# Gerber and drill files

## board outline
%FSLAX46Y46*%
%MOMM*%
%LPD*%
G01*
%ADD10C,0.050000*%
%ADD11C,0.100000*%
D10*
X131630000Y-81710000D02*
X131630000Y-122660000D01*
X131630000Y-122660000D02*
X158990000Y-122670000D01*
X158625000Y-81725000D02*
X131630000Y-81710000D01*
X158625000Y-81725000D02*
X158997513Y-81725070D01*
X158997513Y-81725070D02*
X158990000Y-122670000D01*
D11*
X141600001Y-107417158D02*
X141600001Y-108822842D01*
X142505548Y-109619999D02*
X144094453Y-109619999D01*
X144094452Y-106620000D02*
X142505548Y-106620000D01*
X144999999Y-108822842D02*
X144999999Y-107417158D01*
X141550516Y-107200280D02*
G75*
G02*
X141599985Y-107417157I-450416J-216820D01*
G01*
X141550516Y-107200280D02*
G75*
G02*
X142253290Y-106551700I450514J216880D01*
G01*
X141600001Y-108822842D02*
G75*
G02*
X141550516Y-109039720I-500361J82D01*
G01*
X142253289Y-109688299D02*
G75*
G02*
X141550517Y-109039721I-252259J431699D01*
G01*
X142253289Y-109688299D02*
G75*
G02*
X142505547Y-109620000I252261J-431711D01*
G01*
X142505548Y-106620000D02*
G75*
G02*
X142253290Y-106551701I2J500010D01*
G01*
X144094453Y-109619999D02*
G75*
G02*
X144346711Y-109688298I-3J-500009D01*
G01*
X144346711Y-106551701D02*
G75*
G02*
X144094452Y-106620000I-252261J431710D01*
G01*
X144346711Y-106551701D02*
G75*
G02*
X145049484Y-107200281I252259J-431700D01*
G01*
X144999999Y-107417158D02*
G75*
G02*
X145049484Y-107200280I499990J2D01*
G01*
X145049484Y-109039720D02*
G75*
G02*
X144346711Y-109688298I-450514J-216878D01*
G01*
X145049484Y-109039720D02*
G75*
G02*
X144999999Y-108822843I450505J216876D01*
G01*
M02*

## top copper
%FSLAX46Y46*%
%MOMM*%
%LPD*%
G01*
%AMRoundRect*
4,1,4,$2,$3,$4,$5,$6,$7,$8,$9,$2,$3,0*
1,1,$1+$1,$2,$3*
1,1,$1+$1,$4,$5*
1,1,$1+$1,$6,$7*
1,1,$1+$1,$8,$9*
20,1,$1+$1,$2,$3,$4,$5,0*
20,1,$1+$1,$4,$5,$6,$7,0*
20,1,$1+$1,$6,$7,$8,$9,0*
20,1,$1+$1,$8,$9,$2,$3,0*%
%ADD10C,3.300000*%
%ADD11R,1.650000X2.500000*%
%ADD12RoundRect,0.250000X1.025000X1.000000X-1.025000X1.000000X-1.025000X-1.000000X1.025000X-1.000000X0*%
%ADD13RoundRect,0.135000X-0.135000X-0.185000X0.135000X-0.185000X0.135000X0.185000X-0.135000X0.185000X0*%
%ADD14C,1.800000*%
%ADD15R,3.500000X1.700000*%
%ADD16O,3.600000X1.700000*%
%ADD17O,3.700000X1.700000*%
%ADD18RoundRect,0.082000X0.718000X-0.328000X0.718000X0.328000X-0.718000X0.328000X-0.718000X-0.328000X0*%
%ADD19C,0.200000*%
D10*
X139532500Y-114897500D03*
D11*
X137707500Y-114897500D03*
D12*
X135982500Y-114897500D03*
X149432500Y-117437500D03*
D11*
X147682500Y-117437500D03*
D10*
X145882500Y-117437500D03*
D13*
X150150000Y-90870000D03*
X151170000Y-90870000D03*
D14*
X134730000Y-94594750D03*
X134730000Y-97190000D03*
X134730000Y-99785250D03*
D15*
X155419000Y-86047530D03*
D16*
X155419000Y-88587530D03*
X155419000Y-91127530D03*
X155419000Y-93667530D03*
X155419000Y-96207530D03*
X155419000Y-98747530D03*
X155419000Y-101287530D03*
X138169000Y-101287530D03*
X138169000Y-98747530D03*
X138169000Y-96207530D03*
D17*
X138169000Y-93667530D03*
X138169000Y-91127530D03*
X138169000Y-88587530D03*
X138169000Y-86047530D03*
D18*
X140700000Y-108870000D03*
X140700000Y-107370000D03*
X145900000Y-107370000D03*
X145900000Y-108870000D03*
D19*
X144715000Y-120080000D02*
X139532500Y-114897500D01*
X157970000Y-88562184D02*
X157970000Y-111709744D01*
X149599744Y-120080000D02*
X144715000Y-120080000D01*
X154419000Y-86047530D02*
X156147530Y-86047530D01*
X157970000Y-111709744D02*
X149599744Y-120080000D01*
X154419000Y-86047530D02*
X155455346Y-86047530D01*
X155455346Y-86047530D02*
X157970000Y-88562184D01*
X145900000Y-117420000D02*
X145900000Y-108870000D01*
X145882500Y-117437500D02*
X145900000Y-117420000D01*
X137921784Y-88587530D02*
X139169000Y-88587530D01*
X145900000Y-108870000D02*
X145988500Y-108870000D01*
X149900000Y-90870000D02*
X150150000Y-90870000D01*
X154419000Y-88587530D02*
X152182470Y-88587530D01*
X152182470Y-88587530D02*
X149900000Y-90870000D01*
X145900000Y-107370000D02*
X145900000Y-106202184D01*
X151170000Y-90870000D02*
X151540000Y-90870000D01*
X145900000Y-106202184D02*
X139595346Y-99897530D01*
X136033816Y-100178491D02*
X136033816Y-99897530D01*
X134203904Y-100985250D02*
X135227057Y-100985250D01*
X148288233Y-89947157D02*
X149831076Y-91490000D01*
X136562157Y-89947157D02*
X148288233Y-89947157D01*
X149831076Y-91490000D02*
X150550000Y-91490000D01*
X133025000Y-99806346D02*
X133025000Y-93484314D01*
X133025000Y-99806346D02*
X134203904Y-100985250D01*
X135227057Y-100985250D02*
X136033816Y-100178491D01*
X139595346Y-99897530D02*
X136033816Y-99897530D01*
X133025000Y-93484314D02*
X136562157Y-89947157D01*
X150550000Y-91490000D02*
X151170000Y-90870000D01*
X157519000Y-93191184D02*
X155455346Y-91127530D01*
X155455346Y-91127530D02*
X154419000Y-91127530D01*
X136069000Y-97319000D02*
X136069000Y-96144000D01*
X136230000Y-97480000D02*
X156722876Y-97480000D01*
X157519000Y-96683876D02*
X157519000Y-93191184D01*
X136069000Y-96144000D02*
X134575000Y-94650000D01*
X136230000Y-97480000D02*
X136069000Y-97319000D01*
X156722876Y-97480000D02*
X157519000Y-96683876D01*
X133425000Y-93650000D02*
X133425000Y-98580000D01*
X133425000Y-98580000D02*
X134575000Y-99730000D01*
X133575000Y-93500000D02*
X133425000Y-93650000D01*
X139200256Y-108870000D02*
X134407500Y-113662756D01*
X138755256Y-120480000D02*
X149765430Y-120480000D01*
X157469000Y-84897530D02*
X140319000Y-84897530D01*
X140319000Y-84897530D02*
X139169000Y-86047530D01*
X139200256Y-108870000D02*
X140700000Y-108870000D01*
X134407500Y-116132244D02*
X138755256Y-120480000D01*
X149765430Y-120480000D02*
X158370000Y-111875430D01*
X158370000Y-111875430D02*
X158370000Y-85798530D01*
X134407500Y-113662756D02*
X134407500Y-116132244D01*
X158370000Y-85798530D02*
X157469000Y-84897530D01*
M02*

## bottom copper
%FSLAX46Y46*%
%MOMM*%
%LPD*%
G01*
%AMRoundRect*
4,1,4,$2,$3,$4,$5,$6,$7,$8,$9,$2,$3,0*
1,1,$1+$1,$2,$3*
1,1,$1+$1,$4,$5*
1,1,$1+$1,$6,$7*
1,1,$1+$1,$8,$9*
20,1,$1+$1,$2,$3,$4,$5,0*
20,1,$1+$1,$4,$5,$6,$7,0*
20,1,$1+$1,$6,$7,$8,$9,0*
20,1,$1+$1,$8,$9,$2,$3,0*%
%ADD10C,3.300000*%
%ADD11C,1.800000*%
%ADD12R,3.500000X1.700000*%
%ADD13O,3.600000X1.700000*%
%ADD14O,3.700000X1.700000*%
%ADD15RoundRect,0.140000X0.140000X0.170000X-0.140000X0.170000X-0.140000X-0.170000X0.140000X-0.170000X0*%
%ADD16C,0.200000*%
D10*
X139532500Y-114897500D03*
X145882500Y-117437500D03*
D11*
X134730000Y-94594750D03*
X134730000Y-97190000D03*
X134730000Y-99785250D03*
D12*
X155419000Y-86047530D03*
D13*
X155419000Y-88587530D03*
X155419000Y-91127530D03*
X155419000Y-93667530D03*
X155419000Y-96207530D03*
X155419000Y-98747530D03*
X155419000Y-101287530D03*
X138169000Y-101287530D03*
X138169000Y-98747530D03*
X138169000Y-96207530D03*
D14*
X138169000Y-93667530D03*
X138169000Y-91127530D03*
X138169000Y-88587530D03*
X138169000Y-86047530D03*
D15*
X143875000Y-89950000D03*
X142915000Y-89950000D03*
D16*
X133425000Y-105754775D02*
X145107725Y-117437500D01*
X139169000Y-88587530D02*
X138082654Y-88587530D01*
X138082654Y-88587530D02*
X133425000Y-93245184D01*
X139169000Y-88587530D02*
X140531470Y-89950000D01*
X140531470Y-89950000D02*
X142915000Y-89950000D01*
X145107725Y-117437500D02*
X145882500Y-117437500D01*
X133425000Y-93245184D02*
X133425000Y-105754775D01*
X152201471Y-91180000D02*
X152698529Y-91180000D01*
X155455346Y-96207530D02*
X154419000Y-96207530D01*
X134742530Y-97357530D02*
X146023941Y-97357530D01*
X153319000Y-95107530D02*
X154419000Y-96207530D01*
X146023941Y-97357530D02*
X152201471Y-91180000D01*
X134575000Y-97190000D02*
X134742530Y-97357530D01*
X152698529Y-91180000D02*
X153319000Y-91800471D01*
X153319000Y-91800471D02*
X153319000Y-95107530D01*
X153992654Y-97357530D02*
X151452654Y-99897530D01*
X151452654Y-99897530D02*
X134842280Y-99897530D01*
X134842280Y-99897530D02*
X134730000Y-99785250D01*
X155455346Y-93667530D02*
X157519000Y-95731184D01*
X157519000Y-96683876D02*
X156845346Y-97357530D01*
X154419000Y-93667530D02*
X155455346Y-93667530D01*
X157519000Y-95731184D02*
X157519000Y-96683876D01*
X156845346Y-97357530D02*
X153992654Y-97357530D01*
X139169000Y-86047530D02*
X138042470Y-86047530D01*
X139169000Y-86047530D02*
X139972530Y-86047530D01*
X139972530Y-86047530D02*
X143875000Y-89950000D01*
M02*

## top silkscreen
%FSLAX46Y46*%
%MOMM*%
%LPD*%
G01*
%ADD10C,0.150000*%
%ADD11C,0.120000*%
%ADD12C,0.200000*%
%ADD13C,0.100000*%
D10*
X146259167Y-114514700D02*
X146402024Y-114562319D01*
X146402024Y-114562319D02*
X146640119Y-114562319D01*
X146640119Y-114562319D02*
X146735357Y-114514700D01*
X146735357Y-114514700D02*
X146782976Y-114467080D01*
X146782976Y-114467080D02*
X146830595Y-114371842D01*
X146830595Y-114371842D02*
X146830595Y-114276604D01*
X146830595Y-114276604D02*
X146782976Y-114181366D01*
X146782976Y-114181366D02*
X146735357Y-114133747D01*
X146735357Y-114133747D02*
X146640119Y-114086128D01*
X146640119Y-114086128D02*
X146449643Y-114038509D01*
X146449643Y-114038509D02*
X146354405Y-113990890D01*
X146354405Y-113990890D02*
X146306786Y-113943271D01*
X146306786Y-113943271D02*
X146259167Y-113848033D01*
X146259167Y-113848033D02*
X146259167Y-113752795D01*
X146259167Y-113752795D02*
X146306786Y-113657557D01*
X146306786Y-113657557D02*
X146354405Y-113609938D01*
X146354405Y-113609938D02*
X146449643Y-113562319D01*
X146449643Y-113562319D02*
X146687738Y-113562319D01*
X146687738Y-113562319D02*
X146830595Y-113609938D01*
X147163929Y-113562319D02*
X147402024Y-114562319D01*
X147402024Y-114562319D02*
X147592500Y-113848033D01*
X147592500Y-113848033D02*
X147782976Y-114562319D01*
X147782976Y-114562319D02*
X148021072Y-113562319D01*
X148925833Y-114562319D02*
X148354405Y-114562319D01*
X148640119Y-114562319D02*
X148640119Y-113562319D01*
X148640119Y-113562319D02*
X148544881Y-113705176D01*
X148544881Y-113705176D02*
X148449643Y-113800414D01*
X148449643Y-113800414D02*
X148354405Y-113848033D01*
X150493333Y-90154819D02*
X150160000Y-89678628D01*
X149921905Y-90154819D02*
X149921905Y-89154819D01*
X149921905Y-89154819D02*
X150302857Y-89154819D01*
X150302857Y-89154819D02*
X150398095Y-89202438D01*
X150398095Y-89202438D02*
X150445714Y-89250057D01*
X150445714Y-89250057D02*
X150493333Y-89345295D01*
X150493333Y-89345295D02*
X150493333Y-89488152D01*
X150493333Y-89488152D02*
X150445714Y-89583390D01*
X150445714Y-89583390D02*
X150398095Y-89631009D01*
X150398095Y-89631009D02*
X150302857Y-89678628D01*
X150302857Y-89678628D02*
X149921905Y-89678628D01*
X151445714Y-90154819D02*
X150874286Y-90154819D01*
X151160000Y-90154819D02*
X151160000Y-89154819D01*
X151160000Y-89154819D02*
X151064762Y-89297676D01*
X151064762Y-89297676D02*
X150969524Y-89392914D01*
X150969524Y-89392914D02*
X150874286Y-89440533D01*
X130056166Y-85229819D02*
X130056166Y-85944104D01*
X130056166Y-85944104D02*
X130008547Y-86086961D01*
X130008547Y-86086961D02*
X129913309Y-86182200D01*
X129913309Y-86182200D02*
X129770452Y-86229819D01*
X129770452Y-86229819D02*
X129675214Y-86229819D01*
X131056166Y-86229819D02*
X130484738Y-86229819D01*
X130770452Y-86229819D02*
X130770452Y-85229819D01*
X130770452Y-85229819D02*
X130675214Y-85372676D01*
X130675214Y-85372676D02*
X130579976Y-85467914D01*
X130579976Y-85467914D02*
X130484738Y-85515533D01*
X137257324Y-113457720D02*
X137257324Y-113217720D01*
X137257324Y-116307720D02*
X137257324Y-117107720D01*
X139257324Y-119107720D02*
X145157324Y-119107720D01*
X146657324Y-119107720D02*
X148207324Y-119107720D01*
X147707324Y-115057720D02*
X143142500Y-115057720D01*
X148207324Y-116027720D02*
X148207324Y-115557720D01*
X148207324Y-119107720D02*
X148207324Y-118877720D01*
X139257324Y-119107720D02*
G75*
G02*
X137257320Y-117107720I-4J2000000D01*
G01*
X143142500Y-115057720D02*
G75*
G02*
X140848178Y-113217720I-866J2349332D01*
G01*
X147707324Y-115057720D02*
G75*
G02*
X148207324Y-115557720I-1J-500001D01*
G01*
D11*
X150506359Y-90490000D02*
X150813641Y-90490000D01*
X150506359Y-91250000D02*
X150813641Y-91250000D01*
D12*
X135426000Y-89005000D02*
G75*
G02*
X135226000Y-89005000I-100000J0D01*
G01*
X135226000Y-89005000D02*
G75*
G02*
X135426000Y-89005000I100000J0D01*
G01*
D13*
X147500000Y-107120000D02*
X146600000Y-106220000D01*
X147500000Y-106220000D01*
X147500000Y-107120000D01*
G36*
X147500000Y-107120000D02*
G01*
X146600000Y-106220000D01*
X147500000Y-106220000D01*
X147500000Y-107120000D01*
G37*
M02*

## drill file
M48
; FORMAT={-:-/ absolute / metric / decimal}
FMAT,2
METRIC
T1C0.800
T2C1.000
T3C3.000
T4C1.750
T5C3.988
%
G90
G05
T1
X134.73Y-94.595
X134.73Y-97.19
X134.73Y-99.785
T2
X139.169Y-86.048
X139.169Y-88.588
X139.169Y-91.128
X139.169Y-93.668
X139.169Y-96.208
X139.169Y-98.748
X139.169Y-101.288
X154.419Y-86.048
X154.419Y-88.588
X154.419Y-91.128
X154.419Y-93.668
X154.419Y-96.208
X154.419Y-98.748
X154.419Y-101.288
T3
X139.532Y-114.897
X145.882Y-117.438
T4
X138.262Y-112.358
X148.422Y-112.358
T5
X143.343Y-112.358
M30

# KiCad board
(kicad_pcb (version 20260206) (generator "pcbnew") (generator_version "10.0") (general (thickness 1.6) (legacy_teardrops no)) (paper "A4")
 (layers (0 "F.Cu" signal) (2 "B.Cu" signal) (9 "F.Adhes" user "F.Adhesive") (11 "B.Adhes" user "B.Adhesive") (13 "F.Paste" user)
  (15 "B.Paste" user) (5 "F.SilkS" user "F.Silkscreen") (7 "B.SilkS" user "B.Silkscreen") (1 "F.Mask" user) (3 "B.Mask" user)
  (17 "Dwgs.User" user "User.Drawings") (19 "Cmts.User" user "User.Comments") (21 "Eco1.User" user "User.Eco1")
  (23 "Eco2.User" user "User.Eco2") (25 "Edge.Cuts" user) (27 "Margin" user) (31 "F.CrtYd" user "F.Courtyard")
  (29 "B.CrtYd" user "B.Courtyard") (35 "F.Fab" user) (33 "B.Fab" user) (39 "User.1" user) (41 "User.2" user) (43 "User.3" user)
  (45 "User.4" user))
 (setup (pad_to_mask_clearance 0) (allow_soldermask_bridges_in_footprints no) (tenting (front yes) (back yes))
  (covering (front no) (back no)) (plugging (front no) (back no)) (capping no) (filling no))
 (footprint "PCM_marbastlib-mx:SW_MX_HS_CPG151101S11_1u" (layer "F.Cu") (at 143.3425 112.3575 180)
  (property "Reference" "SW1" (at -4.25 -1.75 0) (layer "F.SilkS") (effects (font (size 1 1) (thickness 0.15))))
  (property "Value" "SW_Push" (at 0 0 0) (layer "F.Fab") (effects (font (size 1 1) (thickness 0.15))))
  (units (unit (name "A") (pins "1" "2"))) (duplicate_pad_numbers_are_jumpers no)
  (fp_line (start 6.085176 -1.10022) (end 6.085176 -0.86022) (stroke (width 0.15) (type solid)) (layer "F.SilkS"))
  (fp_line (start 6.085176 -3.95022) (end 6.085176 -4.75022) (stroke (width 0.15) (type solid)) (layer "F.SilkS"))
  (fp_line (start 4.085176 -6.75022) (end -1.814824 -6.75022) (stroke (width 0.15) (type solid)) (layer "F.SilkS"))
  (fp_line (start -3.314824 -6.75022) (end -4.864824 -6.75022) (stroke (width 0.15) (type solid)) (layer "F.SilkS"))
  (fp_line (start -4.364824 -2.70022) (end 0.2 -2.70022) (stroke (width 0.15) (type solid)) (layer "F.SilkS"))
  (fp_line (start -4.864824 -3.67022) (end -4.864824 -3.20022) (stroke (width 0.15) (type solid)) (layer "F.SilkS"))
  (fp_line (start -4.864824 -6.75022) (end -4.864824 -6.52022) (stroke (width 0.15) (type solid)) (layer "F.SilkS"))
  (fp_arc (start 4.085176 -6.75022) (mid 5.49939 -6.164434) (end 6.085176 -4.75022) (stroke (width 0.15) (type solid)) (layer "F.SilkS"))
  (fp_arc (start 0.2 -2.70022) (mid 1.670693 -2.183637) (end 2.494322 -0.86022) (stroke (width 0.15) (type solid)) (layer "F.SilkS"))
  (fp_arc (start -4.364824 -2.70022) (mid -4.718377 -2.846667) (end -4.864824 -3.20022) (stroke (width 0.15) (type solid)) (layer "F.SilkS"))
  (pad "" np_thru_hole circle (at -5.08 0 180) (size 1.75 1.75) (drill 1.75) (layers "*.Cu" "*.Mask"))
  (pad "" np_thru_hole circle (at 0 0 180) (size 3.9878 3.9878) (drill 3.9878) (layers "*.Cu" "*.Mask"))
  (pad "" np_thru_hole circle (at 5.08 0 180) (size 1.75 1.75) (drill 1.75) (layers "*.Cu" "*.Mask"))
  (pad "1" thru_hole circle (at 3.81 -2.54 180) (size 3.3 3.3) (drill 3) (layers "*.Cu" "*.Mask") (remove_unused_layers no) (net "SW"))
  (pad "1" smd rect (at 5.635 -2.54) (size 1.65 2.5) (layers "F.Cu") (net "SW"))
  (pad "1" smd roundrect (at 7.36 -2.54 180) (size 2.55 2.5) (layers "F.Cu" "F.Mask" "F.Paste") (roundrect_rratio 0.1) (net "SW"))
  (pad "2" smd roundrect (at -6.09 -5.08 180) (size 2.55 2.5) (layers "F.Cu" "F.Mask" "F.Paste") (roundrect_rratio 0.1) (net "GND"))
  (pad "2" smd rect (at -4.34 -5.08 180) (size 1.65 2.5) (layers "F.Cu") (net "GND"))
  (pad "2" thru_hole circle (at -2.54 -5.08 180) (size 3.3 3.3) (drill 3) (layers "*.Cu" "*.Mask") (remove_unused_layers no) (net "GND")))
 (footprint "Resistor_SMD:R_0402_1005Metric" (layer "F.Cu") (at 150.66 90.87)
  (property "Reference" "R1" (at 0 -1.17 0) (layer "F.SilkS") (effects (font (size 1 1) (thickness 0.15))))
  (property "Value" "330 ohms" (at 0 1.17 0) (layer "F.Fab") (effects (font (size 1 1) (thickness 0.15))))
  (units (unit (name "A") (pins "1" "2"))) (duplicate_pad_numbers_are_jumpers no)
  (fp_line (start -0.153641 -0.38) (end 0.153641 -0.38) (stroke (width 0.12) (type solid)) (layer "F.SilkS"))
  (fp_line (start -0.153641 0.38) (end 0.153641 0.38) (stroke (width 0.12) (type solid)) (layer "F.SilkS"))
  (pad "1" smd roundrect (at -0.51 0) (size 0.54 0.64) (layers "F.Cu" "F.Mask" "F.Paste") (roundrect_rratio 0.25) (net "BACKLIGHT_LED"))
  (pad "2" smd roundrect (at 0.51 0) (size 0.54 0.64) (layers "F.Cu" "F.Mask" "F.Paste") (roundrect_rratio 0.25) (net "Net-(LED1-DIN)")))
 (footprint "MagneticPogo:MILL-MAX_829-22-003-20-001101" (layer "F.Cu") (at 130.73 88.39)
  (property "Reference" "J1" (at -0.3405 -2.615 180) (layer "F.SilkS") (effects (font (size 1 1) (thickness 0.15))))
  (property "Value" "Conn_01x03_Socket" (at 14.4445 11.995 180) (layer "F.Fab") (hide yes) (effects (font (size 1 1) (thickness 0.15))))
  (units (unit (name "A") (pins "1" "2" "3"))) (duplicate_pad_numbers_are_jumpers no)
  (fp_circle (center 4.596 0.615) (end 4.596 0.715) (stroke (width 0.2) (type solid)) (fill no) (layer "F.SilkS"))
  (pad "1" thru_hole circle (at 4 6.20475 270) (size 1.8 1.8) (drill 0.8) (layers "*.Cu" "*.Mask") (remove_unused_layers no)
   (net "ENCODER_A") (solder_mask_margin 0.102))
  (pad "2" thru_hole circle (at 4 8.8 270) (size 1.8 1.8) (drill 0.8) (layers "*.Cu" "*.Mask") (remove_unused_layers no) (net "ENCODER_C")
   (solder_mask_margin 0.102))
  (pad "3" thru_hole circle (at 4 11.39525 270) (size 1.8 1.8) (drill 0.8) (layers "*.Cu" "*.Mask") (remove_unused_layers no)
   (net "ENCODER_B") (solder_mask_margin 0.102)))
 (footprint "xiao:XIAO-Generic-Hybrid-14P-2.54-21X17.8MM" (layer "B.Cu") (at 146.794 93.66753 180)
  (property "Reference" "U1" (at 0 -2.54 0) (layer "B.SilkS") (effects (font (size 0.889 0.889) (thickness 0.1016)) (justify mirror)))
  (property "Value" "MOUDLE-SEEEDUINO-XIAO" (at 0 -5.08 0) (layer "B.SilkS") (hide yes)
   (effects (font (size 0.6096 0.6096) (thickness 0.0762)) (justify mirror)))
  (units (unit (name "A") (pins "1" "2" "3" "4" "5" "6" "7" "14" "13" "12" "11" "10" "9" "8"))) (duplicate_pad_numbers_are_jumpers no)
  (pad "1" thru_hole rect (at -7.625 7.62 180) (size 3.5 1.7) (drill 1 (offset -1 0)) (layers "*.Cu" "*.Mask") (remove_unused_layers no)
   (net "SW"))
  (pad "2" thru_hole oval (at -7.625 5.08 180) (size 3.6 1.7) (drill 1 (offset -1 0)) (layers "*.Cu" "*.Mask") (remove_unused_layers no)
   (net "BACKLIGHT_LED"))
  (pad "3" thru_hole oval (at -7.625 2.54 180) (size 3.6 1.7) (drill 1 (offset -1 0)) (layers "*.Cu" "*.Mask") (remove_unused_layers no)
   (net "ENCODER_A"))
  (pad "4" thru_hole oval (at -7.625 0 180) (size 3.6 1.7) (drill 1 (offset -1 0)) (layers "*.Cu" "*.Mask") (remove_unused_layers no)
   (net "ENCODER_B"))
  (pad "5" thru_hole oval (at -7.625 -2.54 180) (size 3.6 1.7) (drill 1 (offset -1 0)) (layers "*.Cu" "*.Mask") (remove_unused_layers no)
   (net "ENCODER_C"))
  (pad "6" thru_hole oval (at -7.625 -5.08) (size 3.6 1.7) (drill 1 (offset 1 0)) (layers "*.Cu" "*.Mask") (remove_unused_layers no)
   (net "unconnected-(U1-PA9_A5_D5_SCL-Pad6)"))
  (pad "7" thru_hole oval (at -7.625 -7.62 180) (size 3.6 1.7) (drill 1 (offset -1 0)) (layers "*.Cu" "*.Mask") (remove_unused_layers no)
   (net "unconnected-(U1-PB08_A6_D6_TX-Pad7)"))
  (pad "8" thru_hole oval (at 7.625 -7.62 180) (size 3.6 1.7) (drill 1 (offset 1 0)) (layers "*.Cu" "*.Mask") (remove_unused_layers no)
   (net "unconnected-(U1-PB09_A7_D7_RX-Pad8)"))
  (pad "9" thru_hole oval (at 7.625 -5.08 180) (size 3.6 1.7) (drill 1 (offset 1 0)) (layers "*.Cu" "*.Mask") (remove_unused_layers no)
   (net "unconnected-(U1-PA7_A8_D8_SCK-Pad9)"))
  (pad "10" thru_hole oval (at 7.625 -2.54 180) (size 3.6 1.7) (drill 1 (offset 1 0)) (layers "*.Cu" "*.Mask") (remove_unused_layers no)
   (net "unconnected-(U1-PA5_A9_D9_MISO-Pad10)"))
  (pad "11" thru_hole oval (at 7.625 0 180) (size 3.7 1.7) (drill 1 (offset 1 0)) (layers "*.Cu" "*.Mask") (remove_unused_layers no)
   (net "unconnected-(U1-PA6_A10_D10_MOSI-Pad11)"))
  (pad "12" thru_hole oval (at 7.625 2.54 180) (size 3.7 1.7) (drill 1 (offset 1 0)) (layers "*.Cu" "*.Mask") (remove_unused_layers no)
   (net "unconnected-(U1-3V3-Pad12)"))
  (pad "13" thru_hole oval (at 7.625 5.08 180) (size 3.7 1.7) (drill 1 (offset 1 0)) (layers "*.Cu" "*.Mask") (remove_unused_layers no)
   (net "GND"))
  (pad "14" thru_hole oval (at 7.625 7.62 180) (size 3.7 1.7) (drill 1 (offset 1 0)) (layers "*.Cu" "*.Mask") (remove_unused_layers no)
   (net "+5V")))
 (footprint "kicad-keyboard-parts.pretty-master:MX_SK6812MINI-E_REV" (layer "B.Cu") (at 143.3 103.04 180)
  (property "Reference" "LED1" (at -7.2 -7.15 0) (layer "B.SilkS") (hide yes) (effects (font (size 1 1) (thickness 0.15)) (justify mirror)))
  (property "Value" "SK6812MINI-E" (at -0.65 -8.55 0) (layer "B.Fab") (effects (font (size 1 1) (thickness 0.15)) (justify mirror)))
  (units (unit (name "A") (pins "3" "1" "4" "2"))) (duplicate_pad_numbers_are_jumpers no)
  (fp_poly (pts (xy -4.2 -4.08) (xy -3.3 -3.18) (xy -4.2 -3.18)) (stroke (width 0.1) (type solid)) (fill yes) (layer "F.SilkS"))
  (fp_line (start 1.699999 -4.377158) (end 1.699999 -5.782842) (stroke (width 0.1) (type solid)) (layer "Edge.Cuts"))
  (fp_line (start 0.794452 -6.579999) (end -0.794453 -6.579999) (stroke (width 0.1) (type solid)) (layer "Edge.Cuts"))
  (fp_line (start -0.794452 -3.58) (end 0.794452 -3.58) (stroke (width 0.1) (type solid)) (layer "Edge.Cuts"))
  (fp_line (start -1.699999 -5.782842) (end -1.699999 -4.377158) (stroke (width 0.1) (type solid)) (layer "Edge.Cuts"))
  (fp_arc (start 1.749484 -4.16028) (mid 1.712526 -4.265931) (end 1.699999 -4.377157) (stroke (width 0.1) (type solid)) (layer "Edge.Cuts"))
  (fp_arc (start 1.749484 -4.16028) (mid 1.638072 -3.575963) (end 1.046711 -3.511703) (stroke (width 0.1) (type solid)) (layer "Edge.Cuts"))
  (fp_arc (start 1.699999 -5.782842) (mid 1.712536 -5.894065) (end 1.749484 -5.99972) (stroke (width 0.1) (type solid)) (layer "Edge.Cuts"))
  (fp_arc (start 1.046711 -6.648299) (mid 1.638071 -6.584036) (end 1.749484 -5.99972) (stroke (width 0.1) (type solid)) (layer "Edge.Cuts"))
  (fp_arc (start 1.046711 -6.648299) (mid 0.925123 -6.597377) (end 0.794453 -6.58) (stroke (width 0.1) (type solid)) (layer "Edge.Cuts"))
  (fp_arc (start 0.794452 -3.58) (mid 0.925122 -3.562623) (end 1.04671 -3.511701) (stroke (width 0.1) (type solid)) (layer "Edge.Cuts"))
  (fp_arc (start -0.794453 -6.579999) (mid -0.925123 -6.597376) (end -1.046711 -6.648298) (stroke (width 0.1) (type solid))
   (layer "Edge.Cuts"))
  (fp_arc (start -1.046711 -3.511701) (mid -0.925123 -3.562623) (end -0.794452 -3.58) (stroke (width 0.1) (type solid)) (layer "Edge.Cuts"))
  (fp_arc (start -1.046711 -3.511701) (mid -1.638072 -3.575965) (end -1.749484 -4.160281) (stroke (width 0.1) (type solid))
   (layer "Edge.Cuts"))
  (fp_arc (start -1.699999 -4.377158) (mid -1.712527 -4.265932) (end -1.749484 -4.16028) (stroke (width 0.1) (type solid))
   (layer "Edge.Cuts"))
  (fp_arc (start -1.749484 -5.99972) (mid -1.638071 -6.584035) (end -1.046711 -6.648298) (stroke (width 0.1) (type solid))
   (layer "Edge.Cuts"))
  (fp_arc (start -1.749484 -5.99972) (mid -1.712527 -5.894068) (end -1.699999 -5.782843) (stroke (width 0.1) (type solid))
   (layer "Edge.Cuts"))
  (pad "1" smd roundrect (at 2.6 -5.83 90) (size 0.82 1.6) (layers "F.Cu" "F.Mask" "F.Paste") (roundrect_rratio 0.1) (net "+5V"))
  (pad "2" smd roundrect (at 2.6 -4.33 90) (size 0.82 1.6) (layers "F.Cu" "F.Mask" "F.Paste") (roundrect_rratio 0.1)
   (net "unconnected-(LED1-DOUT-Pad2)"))
  (pad "3" smd roundrect (at -2.6 -4.33 90) (size 0.82 1.6) (layers "F.Cu" "F.Mask" "F.Paste") (roundrect_rratio 0.1) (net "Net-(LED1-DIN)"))
  (pad "4" smd roundrect (at -2.6 -5.83 90) (size 0.82 1.6) (layers "F.Cu" "F.Mask" "F.Paste") (roundrect_rratio 0.1) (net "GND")))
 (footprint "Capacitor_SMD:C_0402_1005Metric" (layer "B.Cu") (at 143.395 89.95 180)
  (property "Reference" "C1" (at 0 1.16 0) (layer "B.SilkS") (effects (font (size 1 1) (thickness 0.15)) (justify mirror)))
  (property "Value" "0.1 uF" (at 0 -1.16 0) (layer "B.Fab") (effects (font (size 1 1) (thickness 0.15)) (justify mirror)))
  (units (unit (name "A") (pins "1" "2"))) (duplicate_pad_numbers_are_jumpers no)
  (pad "1" smd roundrect (at -0.48 0 180) (size 0.56 0.62) (layers "B.Cu" "B.Mask" "B.Paste") (roundrect_rratio 0.25) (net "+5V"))
  (pad "2" smd roundrect (at 0.48 0 180) (size 0.56 0.62) (layers "B.Cu" "B.Mask" "B.Paste") (roundrect_rratio 0.25) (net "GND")))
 (gr_line (start 131.63 81.71) (end 131.63 122.66) (stroke (width 0.05) (type default)) (layer "Edge.Cuts"))
 (gr_line (start 131.63 122.66) (end 158.99 122.67) (stroke (width 0.05) (type default)) (layer "Edge.Cuts"))
 (gr_line (start 158.625 81.725) (end 131.63 81.71) (stroke (width 0.05) (type default)) (layer "Edge.Cuts"))
 (gr_line (start 158.625 81.725) (end 158.997513 81.72507) (stroke (width 0.05) (type default)) (layer "Edge.Cuts"))
 (gr_line (start 158.997513 81.72507) (end 158.99 122.67) (stroke (width 0.05) (type default)) (layer "Edge.Cuts"))
 (segment (start 144.715 120.08) (end 139.5325 114.8975) (width 0.2) (layer "F.Cu") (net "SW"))
 (segment (start 157.97 88.562184) (end 157.97 111.709744) (width 0.2) (layer "F.Cu") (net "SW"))
 (segment (start 149.599744 120.08) (end 144.715 120.08) (width 0.2) (layer "F.Cu") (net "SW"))
 (segment (start 154.419 86.04753) (end 156.14753 86.04753) (width 0.2) (layer "F.Cu") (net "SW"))
 (segment (start 157.97 111.709744) (end 149.599744 120.08) (width 0.2) (layer "F.Cu") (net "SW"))
 (segment (start 154.419 86.04753) (end 155.455346 86.04753) (width 0.2) (layer "F.Cu") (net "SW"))
 (segment (start 155.455346 86.04753) (end 157.97 88.562184) (width 0.2) (layer "F.Cu") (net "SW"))
 (segment (start 145.9 117.42) (end 145.9 108.87) (width 0.2) (layer "F.Cu") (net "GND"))
 (segment (start 145.8825 117.4375) (end 145.9 117.42) (width 0.2) (layer "F.Cu") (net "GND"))
 (segment (start 137.921784 88.58753) (end 139.169 88.58753) (width 0.2) (layer "F.Cu") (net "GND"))
 (segment (start 145.9 108.87) (end 145.9885 108.87) (width 0.2) (layer "F.Cu") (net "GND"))
 (segment (start 133.425 105.754775) (end 145.107725 117.4375) (width 0.2) (layer "B.Cu") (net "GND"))
 (segment (start 139.169 88.58753) (end 138.082654 88.58753) (width 0.2) (layer "B.Cu") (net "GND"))
 (segment (start 138.082654 88.58753) (end 133.425 93.245184) (width 0.2) (layer "B.Cu") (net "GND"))
 (segment (start 139.169 88.58753) (end 140.53147 89.95) (width 0.2) (layer "B.Cu") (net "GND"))
 (segment (start 140.53147 89.95) (end 142.915 89.95) (width 0.2) (layer "B.Cu") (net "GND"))
 (segment (start 145.107725 117.4375) (end 145.8825 117.4375) (width 0.2) (layer "B.Cu") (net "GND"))
 (segment (start 133.425 93.245184) (end 133.425 105.754775) (width 0.2) (layer "B.Cu") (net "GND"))
 (segment (start 149.9 90.87) (end 150.15 90.87) (width 0.2) (layer "F.Cu") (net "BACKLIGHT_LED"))
 (segment (start 154.419 88.58753) (end 152.18247 88.58753) (width 0.2) (layer "F.Cu") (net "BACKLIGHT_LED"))
 (segment (start 152.18247 88.58753) (end 149.9 90.87) (width 0.2) (layer "F.Cu") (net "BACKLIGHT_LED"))
 (segment (start 145.9 107.37) (end 145.9 106.202184) (width 0.2) (layer "F.Cu") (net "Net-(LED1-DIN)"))
 (segment (start 151.17 90.87) (end 151.54 90.87) (width 0.2) (layer "F.Cu") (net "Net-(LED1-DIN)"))
 (segment (start 145.9 106.202184) (end 139.595346 99.89753) (width 0.2) (layer "F.Cu") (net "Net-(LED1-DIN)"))
 (segment (start 136.033816 100.178491) (end 136.033816 99.89753) (width 0.2) (layer "F.Cu") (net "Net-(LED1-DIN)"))
 (segment (start 134.203904 100.98525) (end 135.227057 100.98525) (width 0.2) (layer "F.Cu") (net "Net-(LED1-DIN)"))
 (segment (start 148.288233 89.947157) (end 149.831076 91.49) (width 0.2) (layer "F.Cu") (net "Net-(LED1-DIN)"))
 (segment (start 136.562157 89.947157) (end 148.288233 89.947157) (width 0.2) (layer "F.Cu") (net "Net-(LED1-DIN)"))
 (segment (start 149.831076 91.49) (end 150.55 91.49) (width 0.2) (layer "F.Cu") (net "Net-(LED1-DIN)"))
 (segment (start 133.025 99.806346) (end 133.025 93.484314) (width 0.2) (layer "F.Cu") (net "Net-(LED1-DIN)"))
 (segment (start 133.025 99.806346) (end 134.203904 100.98525) (width 0.2) (layer "F.Cu") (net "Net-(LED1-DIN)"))
 (segment (start 135.227057 100.98525) (end 136.033816 100.178491) (width 0.2) (layer "F.Cu") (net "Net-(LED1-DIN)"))
 (segment (start 139.595346 99.89753) (end 136.033816 99.89753) (width 0.2) (layer "F.Cu") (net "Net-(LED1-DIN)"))
 (segment (start 133.025 93.484314) (end 136.562157 89.947157) (width 0.2) (layer "F.Cu") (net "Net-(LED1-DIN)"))
 (segment (start 150.55 91.49) (end 151.17 90.87) (width 0.2) (layer "F.Cu") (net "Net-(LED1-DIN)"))
 (segment (start 157.519 93.191184) (end 155.455346 91.12753) (width 0.2) (layer "F.Cu") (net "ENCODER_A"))
 (segment (start 155.455346 91.12753) (end 154.419 91.12753) (width 0.2) (layer "F.Cu") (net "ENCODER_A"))
 (segment (start 136.069 97.319) (end 136.069 96.144) (width 0.2) (layer "F.Cu") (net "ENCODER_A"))
 (segment (start 136.23 97.48) (end 156.722876 97.48) (width 0.2) (layer "F.Cu") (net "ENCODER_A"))
 (segment (start 157.519 96.683876) (end 157.519 93.191184) (width 0.2) (layer "F.Cu") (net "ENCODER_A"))
 (segment (start 136.069 96.144) (end 134.575 94.65) (width 0.2) (layer "F.Cu") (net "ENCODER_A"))
 (segment (start 136.23 97.48) (end 136.069 97.319) (width 0.2) (layer "F.Cu") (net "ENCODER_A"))
 (segment (start 156.722876 97.48) (end 157.519 96.683876) (width 0.2) (layer "F.Cu") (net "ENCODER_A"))
 (segment (start 152.201471 91.18) (end 152.698529 91.18) (width 0.2) (layer "B.Cu") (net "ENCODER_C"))
 (segment (start 155.455346 96.20753) (end 154.419 96.20753) (width 0.2) (layer "B.Cu") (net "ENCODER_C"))
 (segment (start 134.74253 97.35753) (end 146.023941 97.35753) (width 0.2) (layer "B.Cu") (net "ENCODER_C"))
 (segment (start 153.319 95.10753) (end 154.419 96.20753) (width 0.2) (layer "B.Cu") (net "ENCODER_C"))
 (segment (start 146.023941 97.35753) (end 152.201471 91.18) (width 0.2) (layer "B.Cu") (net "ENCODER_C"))
 (segment (start 134.575 97.19) (end 134.74253 97.35753) (width 0.2) (layer "B.Cu") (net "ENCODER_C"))
 (segment (start 152.698529 91.18) (end 153.319 91.800471) (width 0.2) (layer "B.Cu") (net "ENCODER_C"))
 (segment (start 153.319 91.800471) (end 153.319 95.10753) (width 0.2) (layer "B.Cu") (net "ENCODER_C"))
 (segment (start 133.425 93.65) (end 133.425 98.58) (width 0.2) (layer "F.Cu") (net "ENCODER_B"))
 (segment (start 133.425 98.58) (end 134.575 99.73) (width 0.2) (layer "F.Cu") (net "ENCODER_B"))
 (segment (start 133.575 93.5) (end 133.425 93.65) (width 0.2) (layer "F.Cu") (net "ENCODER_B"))
 (segment (start 153.992654 97.35753) (end 151.452654 99.89753) (width 0.2) (layer "B.Cu") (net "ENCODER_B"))
 (segment (start 151.452654 99.89753) (end 134.84228 99.89753) (width 0.2) (layer "B.Cu") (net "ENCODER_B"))
 (segment (start 134.84228 99.89753) (end 134.73 99.78525) (width 0.2) (layer "B.Cu") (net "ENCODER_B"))
 (segment (start 155.455346 93.66753) (end 157.519 95.731184) (width 0.2) (layer "B.Cu") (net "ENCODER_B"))
 (segment (start 157.519 96.683876) (end 156.845346 97.35753) (width 0.2) (layer "B.Cu") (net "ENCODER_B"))
 (segment (start 154.419 93.66753) (end 155.455346 93.66753) (width 0.2) (layer "B.Cu") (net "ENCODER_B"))
 (segment (start 157.519 95.731184) (end 157.519 96.683876) (width 0.2) (layer "B.Cu") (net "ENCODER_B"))
 (segment (start 156.845346 97.35753) (end 153.992654 97.35753) (width 0.2) (layer "B.Cu") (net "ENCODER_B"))
 (segment (start 139.200256 108.87) (end 134.4075 113.662756) (width 0.2) (layer "F.Cu") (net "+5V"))
 (segment (start 138.755256 120.48) (end 149.76543 120.48) (width 0.2) (layer "F.Cu") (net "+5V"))
 (segment (start 157.469 84.89753) (end 140.319 84.89753) (width 0.2) (layer "F.Cu") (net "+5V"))
 (segment (start 140.319 84.89753) (end 139.169 86.04753) (width 0.2) (layer "F.Cu") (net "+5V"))
 (segment (start 139.200256 108.87) (end 140.7 108.87) (width 0.2) (layer "F.Cu") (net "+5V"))
 (segment (start 134.4075 116.132244) (end 138.755256 120.48) (width 0.2) (layer "F.Cu") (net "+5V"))
 (segment (start 149.76543 120.48) (end 158.37 111.87543) (width 0.2) (layer "F.Cu") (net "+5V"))
 (segment (start 158.37 111.87543) (end 158.37 85.79853) (width 0.2) (layer "F.Cu") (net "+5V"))
 (segment (start 134.4075 113.662756) (end 134.4075 116.132244) (width 0.2) (layer "F.Cu") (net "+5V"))
 (segment (start 158.37 85.79853) (end 157.469 84.89753) (width 0.2) (layer "F.Cu") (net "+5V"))
 (segment (start 139.169 86.04753) (end 138.04247 86.04753) (width 0.2) (layer "B.Cu") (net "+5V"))
 (segment (start 139.169 86.04753) (end 139.97253 86.04753) (width 0.2) (layer "B.Cu") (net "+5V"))
 (segment (start 139.97253 86.04753) (end 143.875 89.95) (width 0.2) (layer "B.Cu") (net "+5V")))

